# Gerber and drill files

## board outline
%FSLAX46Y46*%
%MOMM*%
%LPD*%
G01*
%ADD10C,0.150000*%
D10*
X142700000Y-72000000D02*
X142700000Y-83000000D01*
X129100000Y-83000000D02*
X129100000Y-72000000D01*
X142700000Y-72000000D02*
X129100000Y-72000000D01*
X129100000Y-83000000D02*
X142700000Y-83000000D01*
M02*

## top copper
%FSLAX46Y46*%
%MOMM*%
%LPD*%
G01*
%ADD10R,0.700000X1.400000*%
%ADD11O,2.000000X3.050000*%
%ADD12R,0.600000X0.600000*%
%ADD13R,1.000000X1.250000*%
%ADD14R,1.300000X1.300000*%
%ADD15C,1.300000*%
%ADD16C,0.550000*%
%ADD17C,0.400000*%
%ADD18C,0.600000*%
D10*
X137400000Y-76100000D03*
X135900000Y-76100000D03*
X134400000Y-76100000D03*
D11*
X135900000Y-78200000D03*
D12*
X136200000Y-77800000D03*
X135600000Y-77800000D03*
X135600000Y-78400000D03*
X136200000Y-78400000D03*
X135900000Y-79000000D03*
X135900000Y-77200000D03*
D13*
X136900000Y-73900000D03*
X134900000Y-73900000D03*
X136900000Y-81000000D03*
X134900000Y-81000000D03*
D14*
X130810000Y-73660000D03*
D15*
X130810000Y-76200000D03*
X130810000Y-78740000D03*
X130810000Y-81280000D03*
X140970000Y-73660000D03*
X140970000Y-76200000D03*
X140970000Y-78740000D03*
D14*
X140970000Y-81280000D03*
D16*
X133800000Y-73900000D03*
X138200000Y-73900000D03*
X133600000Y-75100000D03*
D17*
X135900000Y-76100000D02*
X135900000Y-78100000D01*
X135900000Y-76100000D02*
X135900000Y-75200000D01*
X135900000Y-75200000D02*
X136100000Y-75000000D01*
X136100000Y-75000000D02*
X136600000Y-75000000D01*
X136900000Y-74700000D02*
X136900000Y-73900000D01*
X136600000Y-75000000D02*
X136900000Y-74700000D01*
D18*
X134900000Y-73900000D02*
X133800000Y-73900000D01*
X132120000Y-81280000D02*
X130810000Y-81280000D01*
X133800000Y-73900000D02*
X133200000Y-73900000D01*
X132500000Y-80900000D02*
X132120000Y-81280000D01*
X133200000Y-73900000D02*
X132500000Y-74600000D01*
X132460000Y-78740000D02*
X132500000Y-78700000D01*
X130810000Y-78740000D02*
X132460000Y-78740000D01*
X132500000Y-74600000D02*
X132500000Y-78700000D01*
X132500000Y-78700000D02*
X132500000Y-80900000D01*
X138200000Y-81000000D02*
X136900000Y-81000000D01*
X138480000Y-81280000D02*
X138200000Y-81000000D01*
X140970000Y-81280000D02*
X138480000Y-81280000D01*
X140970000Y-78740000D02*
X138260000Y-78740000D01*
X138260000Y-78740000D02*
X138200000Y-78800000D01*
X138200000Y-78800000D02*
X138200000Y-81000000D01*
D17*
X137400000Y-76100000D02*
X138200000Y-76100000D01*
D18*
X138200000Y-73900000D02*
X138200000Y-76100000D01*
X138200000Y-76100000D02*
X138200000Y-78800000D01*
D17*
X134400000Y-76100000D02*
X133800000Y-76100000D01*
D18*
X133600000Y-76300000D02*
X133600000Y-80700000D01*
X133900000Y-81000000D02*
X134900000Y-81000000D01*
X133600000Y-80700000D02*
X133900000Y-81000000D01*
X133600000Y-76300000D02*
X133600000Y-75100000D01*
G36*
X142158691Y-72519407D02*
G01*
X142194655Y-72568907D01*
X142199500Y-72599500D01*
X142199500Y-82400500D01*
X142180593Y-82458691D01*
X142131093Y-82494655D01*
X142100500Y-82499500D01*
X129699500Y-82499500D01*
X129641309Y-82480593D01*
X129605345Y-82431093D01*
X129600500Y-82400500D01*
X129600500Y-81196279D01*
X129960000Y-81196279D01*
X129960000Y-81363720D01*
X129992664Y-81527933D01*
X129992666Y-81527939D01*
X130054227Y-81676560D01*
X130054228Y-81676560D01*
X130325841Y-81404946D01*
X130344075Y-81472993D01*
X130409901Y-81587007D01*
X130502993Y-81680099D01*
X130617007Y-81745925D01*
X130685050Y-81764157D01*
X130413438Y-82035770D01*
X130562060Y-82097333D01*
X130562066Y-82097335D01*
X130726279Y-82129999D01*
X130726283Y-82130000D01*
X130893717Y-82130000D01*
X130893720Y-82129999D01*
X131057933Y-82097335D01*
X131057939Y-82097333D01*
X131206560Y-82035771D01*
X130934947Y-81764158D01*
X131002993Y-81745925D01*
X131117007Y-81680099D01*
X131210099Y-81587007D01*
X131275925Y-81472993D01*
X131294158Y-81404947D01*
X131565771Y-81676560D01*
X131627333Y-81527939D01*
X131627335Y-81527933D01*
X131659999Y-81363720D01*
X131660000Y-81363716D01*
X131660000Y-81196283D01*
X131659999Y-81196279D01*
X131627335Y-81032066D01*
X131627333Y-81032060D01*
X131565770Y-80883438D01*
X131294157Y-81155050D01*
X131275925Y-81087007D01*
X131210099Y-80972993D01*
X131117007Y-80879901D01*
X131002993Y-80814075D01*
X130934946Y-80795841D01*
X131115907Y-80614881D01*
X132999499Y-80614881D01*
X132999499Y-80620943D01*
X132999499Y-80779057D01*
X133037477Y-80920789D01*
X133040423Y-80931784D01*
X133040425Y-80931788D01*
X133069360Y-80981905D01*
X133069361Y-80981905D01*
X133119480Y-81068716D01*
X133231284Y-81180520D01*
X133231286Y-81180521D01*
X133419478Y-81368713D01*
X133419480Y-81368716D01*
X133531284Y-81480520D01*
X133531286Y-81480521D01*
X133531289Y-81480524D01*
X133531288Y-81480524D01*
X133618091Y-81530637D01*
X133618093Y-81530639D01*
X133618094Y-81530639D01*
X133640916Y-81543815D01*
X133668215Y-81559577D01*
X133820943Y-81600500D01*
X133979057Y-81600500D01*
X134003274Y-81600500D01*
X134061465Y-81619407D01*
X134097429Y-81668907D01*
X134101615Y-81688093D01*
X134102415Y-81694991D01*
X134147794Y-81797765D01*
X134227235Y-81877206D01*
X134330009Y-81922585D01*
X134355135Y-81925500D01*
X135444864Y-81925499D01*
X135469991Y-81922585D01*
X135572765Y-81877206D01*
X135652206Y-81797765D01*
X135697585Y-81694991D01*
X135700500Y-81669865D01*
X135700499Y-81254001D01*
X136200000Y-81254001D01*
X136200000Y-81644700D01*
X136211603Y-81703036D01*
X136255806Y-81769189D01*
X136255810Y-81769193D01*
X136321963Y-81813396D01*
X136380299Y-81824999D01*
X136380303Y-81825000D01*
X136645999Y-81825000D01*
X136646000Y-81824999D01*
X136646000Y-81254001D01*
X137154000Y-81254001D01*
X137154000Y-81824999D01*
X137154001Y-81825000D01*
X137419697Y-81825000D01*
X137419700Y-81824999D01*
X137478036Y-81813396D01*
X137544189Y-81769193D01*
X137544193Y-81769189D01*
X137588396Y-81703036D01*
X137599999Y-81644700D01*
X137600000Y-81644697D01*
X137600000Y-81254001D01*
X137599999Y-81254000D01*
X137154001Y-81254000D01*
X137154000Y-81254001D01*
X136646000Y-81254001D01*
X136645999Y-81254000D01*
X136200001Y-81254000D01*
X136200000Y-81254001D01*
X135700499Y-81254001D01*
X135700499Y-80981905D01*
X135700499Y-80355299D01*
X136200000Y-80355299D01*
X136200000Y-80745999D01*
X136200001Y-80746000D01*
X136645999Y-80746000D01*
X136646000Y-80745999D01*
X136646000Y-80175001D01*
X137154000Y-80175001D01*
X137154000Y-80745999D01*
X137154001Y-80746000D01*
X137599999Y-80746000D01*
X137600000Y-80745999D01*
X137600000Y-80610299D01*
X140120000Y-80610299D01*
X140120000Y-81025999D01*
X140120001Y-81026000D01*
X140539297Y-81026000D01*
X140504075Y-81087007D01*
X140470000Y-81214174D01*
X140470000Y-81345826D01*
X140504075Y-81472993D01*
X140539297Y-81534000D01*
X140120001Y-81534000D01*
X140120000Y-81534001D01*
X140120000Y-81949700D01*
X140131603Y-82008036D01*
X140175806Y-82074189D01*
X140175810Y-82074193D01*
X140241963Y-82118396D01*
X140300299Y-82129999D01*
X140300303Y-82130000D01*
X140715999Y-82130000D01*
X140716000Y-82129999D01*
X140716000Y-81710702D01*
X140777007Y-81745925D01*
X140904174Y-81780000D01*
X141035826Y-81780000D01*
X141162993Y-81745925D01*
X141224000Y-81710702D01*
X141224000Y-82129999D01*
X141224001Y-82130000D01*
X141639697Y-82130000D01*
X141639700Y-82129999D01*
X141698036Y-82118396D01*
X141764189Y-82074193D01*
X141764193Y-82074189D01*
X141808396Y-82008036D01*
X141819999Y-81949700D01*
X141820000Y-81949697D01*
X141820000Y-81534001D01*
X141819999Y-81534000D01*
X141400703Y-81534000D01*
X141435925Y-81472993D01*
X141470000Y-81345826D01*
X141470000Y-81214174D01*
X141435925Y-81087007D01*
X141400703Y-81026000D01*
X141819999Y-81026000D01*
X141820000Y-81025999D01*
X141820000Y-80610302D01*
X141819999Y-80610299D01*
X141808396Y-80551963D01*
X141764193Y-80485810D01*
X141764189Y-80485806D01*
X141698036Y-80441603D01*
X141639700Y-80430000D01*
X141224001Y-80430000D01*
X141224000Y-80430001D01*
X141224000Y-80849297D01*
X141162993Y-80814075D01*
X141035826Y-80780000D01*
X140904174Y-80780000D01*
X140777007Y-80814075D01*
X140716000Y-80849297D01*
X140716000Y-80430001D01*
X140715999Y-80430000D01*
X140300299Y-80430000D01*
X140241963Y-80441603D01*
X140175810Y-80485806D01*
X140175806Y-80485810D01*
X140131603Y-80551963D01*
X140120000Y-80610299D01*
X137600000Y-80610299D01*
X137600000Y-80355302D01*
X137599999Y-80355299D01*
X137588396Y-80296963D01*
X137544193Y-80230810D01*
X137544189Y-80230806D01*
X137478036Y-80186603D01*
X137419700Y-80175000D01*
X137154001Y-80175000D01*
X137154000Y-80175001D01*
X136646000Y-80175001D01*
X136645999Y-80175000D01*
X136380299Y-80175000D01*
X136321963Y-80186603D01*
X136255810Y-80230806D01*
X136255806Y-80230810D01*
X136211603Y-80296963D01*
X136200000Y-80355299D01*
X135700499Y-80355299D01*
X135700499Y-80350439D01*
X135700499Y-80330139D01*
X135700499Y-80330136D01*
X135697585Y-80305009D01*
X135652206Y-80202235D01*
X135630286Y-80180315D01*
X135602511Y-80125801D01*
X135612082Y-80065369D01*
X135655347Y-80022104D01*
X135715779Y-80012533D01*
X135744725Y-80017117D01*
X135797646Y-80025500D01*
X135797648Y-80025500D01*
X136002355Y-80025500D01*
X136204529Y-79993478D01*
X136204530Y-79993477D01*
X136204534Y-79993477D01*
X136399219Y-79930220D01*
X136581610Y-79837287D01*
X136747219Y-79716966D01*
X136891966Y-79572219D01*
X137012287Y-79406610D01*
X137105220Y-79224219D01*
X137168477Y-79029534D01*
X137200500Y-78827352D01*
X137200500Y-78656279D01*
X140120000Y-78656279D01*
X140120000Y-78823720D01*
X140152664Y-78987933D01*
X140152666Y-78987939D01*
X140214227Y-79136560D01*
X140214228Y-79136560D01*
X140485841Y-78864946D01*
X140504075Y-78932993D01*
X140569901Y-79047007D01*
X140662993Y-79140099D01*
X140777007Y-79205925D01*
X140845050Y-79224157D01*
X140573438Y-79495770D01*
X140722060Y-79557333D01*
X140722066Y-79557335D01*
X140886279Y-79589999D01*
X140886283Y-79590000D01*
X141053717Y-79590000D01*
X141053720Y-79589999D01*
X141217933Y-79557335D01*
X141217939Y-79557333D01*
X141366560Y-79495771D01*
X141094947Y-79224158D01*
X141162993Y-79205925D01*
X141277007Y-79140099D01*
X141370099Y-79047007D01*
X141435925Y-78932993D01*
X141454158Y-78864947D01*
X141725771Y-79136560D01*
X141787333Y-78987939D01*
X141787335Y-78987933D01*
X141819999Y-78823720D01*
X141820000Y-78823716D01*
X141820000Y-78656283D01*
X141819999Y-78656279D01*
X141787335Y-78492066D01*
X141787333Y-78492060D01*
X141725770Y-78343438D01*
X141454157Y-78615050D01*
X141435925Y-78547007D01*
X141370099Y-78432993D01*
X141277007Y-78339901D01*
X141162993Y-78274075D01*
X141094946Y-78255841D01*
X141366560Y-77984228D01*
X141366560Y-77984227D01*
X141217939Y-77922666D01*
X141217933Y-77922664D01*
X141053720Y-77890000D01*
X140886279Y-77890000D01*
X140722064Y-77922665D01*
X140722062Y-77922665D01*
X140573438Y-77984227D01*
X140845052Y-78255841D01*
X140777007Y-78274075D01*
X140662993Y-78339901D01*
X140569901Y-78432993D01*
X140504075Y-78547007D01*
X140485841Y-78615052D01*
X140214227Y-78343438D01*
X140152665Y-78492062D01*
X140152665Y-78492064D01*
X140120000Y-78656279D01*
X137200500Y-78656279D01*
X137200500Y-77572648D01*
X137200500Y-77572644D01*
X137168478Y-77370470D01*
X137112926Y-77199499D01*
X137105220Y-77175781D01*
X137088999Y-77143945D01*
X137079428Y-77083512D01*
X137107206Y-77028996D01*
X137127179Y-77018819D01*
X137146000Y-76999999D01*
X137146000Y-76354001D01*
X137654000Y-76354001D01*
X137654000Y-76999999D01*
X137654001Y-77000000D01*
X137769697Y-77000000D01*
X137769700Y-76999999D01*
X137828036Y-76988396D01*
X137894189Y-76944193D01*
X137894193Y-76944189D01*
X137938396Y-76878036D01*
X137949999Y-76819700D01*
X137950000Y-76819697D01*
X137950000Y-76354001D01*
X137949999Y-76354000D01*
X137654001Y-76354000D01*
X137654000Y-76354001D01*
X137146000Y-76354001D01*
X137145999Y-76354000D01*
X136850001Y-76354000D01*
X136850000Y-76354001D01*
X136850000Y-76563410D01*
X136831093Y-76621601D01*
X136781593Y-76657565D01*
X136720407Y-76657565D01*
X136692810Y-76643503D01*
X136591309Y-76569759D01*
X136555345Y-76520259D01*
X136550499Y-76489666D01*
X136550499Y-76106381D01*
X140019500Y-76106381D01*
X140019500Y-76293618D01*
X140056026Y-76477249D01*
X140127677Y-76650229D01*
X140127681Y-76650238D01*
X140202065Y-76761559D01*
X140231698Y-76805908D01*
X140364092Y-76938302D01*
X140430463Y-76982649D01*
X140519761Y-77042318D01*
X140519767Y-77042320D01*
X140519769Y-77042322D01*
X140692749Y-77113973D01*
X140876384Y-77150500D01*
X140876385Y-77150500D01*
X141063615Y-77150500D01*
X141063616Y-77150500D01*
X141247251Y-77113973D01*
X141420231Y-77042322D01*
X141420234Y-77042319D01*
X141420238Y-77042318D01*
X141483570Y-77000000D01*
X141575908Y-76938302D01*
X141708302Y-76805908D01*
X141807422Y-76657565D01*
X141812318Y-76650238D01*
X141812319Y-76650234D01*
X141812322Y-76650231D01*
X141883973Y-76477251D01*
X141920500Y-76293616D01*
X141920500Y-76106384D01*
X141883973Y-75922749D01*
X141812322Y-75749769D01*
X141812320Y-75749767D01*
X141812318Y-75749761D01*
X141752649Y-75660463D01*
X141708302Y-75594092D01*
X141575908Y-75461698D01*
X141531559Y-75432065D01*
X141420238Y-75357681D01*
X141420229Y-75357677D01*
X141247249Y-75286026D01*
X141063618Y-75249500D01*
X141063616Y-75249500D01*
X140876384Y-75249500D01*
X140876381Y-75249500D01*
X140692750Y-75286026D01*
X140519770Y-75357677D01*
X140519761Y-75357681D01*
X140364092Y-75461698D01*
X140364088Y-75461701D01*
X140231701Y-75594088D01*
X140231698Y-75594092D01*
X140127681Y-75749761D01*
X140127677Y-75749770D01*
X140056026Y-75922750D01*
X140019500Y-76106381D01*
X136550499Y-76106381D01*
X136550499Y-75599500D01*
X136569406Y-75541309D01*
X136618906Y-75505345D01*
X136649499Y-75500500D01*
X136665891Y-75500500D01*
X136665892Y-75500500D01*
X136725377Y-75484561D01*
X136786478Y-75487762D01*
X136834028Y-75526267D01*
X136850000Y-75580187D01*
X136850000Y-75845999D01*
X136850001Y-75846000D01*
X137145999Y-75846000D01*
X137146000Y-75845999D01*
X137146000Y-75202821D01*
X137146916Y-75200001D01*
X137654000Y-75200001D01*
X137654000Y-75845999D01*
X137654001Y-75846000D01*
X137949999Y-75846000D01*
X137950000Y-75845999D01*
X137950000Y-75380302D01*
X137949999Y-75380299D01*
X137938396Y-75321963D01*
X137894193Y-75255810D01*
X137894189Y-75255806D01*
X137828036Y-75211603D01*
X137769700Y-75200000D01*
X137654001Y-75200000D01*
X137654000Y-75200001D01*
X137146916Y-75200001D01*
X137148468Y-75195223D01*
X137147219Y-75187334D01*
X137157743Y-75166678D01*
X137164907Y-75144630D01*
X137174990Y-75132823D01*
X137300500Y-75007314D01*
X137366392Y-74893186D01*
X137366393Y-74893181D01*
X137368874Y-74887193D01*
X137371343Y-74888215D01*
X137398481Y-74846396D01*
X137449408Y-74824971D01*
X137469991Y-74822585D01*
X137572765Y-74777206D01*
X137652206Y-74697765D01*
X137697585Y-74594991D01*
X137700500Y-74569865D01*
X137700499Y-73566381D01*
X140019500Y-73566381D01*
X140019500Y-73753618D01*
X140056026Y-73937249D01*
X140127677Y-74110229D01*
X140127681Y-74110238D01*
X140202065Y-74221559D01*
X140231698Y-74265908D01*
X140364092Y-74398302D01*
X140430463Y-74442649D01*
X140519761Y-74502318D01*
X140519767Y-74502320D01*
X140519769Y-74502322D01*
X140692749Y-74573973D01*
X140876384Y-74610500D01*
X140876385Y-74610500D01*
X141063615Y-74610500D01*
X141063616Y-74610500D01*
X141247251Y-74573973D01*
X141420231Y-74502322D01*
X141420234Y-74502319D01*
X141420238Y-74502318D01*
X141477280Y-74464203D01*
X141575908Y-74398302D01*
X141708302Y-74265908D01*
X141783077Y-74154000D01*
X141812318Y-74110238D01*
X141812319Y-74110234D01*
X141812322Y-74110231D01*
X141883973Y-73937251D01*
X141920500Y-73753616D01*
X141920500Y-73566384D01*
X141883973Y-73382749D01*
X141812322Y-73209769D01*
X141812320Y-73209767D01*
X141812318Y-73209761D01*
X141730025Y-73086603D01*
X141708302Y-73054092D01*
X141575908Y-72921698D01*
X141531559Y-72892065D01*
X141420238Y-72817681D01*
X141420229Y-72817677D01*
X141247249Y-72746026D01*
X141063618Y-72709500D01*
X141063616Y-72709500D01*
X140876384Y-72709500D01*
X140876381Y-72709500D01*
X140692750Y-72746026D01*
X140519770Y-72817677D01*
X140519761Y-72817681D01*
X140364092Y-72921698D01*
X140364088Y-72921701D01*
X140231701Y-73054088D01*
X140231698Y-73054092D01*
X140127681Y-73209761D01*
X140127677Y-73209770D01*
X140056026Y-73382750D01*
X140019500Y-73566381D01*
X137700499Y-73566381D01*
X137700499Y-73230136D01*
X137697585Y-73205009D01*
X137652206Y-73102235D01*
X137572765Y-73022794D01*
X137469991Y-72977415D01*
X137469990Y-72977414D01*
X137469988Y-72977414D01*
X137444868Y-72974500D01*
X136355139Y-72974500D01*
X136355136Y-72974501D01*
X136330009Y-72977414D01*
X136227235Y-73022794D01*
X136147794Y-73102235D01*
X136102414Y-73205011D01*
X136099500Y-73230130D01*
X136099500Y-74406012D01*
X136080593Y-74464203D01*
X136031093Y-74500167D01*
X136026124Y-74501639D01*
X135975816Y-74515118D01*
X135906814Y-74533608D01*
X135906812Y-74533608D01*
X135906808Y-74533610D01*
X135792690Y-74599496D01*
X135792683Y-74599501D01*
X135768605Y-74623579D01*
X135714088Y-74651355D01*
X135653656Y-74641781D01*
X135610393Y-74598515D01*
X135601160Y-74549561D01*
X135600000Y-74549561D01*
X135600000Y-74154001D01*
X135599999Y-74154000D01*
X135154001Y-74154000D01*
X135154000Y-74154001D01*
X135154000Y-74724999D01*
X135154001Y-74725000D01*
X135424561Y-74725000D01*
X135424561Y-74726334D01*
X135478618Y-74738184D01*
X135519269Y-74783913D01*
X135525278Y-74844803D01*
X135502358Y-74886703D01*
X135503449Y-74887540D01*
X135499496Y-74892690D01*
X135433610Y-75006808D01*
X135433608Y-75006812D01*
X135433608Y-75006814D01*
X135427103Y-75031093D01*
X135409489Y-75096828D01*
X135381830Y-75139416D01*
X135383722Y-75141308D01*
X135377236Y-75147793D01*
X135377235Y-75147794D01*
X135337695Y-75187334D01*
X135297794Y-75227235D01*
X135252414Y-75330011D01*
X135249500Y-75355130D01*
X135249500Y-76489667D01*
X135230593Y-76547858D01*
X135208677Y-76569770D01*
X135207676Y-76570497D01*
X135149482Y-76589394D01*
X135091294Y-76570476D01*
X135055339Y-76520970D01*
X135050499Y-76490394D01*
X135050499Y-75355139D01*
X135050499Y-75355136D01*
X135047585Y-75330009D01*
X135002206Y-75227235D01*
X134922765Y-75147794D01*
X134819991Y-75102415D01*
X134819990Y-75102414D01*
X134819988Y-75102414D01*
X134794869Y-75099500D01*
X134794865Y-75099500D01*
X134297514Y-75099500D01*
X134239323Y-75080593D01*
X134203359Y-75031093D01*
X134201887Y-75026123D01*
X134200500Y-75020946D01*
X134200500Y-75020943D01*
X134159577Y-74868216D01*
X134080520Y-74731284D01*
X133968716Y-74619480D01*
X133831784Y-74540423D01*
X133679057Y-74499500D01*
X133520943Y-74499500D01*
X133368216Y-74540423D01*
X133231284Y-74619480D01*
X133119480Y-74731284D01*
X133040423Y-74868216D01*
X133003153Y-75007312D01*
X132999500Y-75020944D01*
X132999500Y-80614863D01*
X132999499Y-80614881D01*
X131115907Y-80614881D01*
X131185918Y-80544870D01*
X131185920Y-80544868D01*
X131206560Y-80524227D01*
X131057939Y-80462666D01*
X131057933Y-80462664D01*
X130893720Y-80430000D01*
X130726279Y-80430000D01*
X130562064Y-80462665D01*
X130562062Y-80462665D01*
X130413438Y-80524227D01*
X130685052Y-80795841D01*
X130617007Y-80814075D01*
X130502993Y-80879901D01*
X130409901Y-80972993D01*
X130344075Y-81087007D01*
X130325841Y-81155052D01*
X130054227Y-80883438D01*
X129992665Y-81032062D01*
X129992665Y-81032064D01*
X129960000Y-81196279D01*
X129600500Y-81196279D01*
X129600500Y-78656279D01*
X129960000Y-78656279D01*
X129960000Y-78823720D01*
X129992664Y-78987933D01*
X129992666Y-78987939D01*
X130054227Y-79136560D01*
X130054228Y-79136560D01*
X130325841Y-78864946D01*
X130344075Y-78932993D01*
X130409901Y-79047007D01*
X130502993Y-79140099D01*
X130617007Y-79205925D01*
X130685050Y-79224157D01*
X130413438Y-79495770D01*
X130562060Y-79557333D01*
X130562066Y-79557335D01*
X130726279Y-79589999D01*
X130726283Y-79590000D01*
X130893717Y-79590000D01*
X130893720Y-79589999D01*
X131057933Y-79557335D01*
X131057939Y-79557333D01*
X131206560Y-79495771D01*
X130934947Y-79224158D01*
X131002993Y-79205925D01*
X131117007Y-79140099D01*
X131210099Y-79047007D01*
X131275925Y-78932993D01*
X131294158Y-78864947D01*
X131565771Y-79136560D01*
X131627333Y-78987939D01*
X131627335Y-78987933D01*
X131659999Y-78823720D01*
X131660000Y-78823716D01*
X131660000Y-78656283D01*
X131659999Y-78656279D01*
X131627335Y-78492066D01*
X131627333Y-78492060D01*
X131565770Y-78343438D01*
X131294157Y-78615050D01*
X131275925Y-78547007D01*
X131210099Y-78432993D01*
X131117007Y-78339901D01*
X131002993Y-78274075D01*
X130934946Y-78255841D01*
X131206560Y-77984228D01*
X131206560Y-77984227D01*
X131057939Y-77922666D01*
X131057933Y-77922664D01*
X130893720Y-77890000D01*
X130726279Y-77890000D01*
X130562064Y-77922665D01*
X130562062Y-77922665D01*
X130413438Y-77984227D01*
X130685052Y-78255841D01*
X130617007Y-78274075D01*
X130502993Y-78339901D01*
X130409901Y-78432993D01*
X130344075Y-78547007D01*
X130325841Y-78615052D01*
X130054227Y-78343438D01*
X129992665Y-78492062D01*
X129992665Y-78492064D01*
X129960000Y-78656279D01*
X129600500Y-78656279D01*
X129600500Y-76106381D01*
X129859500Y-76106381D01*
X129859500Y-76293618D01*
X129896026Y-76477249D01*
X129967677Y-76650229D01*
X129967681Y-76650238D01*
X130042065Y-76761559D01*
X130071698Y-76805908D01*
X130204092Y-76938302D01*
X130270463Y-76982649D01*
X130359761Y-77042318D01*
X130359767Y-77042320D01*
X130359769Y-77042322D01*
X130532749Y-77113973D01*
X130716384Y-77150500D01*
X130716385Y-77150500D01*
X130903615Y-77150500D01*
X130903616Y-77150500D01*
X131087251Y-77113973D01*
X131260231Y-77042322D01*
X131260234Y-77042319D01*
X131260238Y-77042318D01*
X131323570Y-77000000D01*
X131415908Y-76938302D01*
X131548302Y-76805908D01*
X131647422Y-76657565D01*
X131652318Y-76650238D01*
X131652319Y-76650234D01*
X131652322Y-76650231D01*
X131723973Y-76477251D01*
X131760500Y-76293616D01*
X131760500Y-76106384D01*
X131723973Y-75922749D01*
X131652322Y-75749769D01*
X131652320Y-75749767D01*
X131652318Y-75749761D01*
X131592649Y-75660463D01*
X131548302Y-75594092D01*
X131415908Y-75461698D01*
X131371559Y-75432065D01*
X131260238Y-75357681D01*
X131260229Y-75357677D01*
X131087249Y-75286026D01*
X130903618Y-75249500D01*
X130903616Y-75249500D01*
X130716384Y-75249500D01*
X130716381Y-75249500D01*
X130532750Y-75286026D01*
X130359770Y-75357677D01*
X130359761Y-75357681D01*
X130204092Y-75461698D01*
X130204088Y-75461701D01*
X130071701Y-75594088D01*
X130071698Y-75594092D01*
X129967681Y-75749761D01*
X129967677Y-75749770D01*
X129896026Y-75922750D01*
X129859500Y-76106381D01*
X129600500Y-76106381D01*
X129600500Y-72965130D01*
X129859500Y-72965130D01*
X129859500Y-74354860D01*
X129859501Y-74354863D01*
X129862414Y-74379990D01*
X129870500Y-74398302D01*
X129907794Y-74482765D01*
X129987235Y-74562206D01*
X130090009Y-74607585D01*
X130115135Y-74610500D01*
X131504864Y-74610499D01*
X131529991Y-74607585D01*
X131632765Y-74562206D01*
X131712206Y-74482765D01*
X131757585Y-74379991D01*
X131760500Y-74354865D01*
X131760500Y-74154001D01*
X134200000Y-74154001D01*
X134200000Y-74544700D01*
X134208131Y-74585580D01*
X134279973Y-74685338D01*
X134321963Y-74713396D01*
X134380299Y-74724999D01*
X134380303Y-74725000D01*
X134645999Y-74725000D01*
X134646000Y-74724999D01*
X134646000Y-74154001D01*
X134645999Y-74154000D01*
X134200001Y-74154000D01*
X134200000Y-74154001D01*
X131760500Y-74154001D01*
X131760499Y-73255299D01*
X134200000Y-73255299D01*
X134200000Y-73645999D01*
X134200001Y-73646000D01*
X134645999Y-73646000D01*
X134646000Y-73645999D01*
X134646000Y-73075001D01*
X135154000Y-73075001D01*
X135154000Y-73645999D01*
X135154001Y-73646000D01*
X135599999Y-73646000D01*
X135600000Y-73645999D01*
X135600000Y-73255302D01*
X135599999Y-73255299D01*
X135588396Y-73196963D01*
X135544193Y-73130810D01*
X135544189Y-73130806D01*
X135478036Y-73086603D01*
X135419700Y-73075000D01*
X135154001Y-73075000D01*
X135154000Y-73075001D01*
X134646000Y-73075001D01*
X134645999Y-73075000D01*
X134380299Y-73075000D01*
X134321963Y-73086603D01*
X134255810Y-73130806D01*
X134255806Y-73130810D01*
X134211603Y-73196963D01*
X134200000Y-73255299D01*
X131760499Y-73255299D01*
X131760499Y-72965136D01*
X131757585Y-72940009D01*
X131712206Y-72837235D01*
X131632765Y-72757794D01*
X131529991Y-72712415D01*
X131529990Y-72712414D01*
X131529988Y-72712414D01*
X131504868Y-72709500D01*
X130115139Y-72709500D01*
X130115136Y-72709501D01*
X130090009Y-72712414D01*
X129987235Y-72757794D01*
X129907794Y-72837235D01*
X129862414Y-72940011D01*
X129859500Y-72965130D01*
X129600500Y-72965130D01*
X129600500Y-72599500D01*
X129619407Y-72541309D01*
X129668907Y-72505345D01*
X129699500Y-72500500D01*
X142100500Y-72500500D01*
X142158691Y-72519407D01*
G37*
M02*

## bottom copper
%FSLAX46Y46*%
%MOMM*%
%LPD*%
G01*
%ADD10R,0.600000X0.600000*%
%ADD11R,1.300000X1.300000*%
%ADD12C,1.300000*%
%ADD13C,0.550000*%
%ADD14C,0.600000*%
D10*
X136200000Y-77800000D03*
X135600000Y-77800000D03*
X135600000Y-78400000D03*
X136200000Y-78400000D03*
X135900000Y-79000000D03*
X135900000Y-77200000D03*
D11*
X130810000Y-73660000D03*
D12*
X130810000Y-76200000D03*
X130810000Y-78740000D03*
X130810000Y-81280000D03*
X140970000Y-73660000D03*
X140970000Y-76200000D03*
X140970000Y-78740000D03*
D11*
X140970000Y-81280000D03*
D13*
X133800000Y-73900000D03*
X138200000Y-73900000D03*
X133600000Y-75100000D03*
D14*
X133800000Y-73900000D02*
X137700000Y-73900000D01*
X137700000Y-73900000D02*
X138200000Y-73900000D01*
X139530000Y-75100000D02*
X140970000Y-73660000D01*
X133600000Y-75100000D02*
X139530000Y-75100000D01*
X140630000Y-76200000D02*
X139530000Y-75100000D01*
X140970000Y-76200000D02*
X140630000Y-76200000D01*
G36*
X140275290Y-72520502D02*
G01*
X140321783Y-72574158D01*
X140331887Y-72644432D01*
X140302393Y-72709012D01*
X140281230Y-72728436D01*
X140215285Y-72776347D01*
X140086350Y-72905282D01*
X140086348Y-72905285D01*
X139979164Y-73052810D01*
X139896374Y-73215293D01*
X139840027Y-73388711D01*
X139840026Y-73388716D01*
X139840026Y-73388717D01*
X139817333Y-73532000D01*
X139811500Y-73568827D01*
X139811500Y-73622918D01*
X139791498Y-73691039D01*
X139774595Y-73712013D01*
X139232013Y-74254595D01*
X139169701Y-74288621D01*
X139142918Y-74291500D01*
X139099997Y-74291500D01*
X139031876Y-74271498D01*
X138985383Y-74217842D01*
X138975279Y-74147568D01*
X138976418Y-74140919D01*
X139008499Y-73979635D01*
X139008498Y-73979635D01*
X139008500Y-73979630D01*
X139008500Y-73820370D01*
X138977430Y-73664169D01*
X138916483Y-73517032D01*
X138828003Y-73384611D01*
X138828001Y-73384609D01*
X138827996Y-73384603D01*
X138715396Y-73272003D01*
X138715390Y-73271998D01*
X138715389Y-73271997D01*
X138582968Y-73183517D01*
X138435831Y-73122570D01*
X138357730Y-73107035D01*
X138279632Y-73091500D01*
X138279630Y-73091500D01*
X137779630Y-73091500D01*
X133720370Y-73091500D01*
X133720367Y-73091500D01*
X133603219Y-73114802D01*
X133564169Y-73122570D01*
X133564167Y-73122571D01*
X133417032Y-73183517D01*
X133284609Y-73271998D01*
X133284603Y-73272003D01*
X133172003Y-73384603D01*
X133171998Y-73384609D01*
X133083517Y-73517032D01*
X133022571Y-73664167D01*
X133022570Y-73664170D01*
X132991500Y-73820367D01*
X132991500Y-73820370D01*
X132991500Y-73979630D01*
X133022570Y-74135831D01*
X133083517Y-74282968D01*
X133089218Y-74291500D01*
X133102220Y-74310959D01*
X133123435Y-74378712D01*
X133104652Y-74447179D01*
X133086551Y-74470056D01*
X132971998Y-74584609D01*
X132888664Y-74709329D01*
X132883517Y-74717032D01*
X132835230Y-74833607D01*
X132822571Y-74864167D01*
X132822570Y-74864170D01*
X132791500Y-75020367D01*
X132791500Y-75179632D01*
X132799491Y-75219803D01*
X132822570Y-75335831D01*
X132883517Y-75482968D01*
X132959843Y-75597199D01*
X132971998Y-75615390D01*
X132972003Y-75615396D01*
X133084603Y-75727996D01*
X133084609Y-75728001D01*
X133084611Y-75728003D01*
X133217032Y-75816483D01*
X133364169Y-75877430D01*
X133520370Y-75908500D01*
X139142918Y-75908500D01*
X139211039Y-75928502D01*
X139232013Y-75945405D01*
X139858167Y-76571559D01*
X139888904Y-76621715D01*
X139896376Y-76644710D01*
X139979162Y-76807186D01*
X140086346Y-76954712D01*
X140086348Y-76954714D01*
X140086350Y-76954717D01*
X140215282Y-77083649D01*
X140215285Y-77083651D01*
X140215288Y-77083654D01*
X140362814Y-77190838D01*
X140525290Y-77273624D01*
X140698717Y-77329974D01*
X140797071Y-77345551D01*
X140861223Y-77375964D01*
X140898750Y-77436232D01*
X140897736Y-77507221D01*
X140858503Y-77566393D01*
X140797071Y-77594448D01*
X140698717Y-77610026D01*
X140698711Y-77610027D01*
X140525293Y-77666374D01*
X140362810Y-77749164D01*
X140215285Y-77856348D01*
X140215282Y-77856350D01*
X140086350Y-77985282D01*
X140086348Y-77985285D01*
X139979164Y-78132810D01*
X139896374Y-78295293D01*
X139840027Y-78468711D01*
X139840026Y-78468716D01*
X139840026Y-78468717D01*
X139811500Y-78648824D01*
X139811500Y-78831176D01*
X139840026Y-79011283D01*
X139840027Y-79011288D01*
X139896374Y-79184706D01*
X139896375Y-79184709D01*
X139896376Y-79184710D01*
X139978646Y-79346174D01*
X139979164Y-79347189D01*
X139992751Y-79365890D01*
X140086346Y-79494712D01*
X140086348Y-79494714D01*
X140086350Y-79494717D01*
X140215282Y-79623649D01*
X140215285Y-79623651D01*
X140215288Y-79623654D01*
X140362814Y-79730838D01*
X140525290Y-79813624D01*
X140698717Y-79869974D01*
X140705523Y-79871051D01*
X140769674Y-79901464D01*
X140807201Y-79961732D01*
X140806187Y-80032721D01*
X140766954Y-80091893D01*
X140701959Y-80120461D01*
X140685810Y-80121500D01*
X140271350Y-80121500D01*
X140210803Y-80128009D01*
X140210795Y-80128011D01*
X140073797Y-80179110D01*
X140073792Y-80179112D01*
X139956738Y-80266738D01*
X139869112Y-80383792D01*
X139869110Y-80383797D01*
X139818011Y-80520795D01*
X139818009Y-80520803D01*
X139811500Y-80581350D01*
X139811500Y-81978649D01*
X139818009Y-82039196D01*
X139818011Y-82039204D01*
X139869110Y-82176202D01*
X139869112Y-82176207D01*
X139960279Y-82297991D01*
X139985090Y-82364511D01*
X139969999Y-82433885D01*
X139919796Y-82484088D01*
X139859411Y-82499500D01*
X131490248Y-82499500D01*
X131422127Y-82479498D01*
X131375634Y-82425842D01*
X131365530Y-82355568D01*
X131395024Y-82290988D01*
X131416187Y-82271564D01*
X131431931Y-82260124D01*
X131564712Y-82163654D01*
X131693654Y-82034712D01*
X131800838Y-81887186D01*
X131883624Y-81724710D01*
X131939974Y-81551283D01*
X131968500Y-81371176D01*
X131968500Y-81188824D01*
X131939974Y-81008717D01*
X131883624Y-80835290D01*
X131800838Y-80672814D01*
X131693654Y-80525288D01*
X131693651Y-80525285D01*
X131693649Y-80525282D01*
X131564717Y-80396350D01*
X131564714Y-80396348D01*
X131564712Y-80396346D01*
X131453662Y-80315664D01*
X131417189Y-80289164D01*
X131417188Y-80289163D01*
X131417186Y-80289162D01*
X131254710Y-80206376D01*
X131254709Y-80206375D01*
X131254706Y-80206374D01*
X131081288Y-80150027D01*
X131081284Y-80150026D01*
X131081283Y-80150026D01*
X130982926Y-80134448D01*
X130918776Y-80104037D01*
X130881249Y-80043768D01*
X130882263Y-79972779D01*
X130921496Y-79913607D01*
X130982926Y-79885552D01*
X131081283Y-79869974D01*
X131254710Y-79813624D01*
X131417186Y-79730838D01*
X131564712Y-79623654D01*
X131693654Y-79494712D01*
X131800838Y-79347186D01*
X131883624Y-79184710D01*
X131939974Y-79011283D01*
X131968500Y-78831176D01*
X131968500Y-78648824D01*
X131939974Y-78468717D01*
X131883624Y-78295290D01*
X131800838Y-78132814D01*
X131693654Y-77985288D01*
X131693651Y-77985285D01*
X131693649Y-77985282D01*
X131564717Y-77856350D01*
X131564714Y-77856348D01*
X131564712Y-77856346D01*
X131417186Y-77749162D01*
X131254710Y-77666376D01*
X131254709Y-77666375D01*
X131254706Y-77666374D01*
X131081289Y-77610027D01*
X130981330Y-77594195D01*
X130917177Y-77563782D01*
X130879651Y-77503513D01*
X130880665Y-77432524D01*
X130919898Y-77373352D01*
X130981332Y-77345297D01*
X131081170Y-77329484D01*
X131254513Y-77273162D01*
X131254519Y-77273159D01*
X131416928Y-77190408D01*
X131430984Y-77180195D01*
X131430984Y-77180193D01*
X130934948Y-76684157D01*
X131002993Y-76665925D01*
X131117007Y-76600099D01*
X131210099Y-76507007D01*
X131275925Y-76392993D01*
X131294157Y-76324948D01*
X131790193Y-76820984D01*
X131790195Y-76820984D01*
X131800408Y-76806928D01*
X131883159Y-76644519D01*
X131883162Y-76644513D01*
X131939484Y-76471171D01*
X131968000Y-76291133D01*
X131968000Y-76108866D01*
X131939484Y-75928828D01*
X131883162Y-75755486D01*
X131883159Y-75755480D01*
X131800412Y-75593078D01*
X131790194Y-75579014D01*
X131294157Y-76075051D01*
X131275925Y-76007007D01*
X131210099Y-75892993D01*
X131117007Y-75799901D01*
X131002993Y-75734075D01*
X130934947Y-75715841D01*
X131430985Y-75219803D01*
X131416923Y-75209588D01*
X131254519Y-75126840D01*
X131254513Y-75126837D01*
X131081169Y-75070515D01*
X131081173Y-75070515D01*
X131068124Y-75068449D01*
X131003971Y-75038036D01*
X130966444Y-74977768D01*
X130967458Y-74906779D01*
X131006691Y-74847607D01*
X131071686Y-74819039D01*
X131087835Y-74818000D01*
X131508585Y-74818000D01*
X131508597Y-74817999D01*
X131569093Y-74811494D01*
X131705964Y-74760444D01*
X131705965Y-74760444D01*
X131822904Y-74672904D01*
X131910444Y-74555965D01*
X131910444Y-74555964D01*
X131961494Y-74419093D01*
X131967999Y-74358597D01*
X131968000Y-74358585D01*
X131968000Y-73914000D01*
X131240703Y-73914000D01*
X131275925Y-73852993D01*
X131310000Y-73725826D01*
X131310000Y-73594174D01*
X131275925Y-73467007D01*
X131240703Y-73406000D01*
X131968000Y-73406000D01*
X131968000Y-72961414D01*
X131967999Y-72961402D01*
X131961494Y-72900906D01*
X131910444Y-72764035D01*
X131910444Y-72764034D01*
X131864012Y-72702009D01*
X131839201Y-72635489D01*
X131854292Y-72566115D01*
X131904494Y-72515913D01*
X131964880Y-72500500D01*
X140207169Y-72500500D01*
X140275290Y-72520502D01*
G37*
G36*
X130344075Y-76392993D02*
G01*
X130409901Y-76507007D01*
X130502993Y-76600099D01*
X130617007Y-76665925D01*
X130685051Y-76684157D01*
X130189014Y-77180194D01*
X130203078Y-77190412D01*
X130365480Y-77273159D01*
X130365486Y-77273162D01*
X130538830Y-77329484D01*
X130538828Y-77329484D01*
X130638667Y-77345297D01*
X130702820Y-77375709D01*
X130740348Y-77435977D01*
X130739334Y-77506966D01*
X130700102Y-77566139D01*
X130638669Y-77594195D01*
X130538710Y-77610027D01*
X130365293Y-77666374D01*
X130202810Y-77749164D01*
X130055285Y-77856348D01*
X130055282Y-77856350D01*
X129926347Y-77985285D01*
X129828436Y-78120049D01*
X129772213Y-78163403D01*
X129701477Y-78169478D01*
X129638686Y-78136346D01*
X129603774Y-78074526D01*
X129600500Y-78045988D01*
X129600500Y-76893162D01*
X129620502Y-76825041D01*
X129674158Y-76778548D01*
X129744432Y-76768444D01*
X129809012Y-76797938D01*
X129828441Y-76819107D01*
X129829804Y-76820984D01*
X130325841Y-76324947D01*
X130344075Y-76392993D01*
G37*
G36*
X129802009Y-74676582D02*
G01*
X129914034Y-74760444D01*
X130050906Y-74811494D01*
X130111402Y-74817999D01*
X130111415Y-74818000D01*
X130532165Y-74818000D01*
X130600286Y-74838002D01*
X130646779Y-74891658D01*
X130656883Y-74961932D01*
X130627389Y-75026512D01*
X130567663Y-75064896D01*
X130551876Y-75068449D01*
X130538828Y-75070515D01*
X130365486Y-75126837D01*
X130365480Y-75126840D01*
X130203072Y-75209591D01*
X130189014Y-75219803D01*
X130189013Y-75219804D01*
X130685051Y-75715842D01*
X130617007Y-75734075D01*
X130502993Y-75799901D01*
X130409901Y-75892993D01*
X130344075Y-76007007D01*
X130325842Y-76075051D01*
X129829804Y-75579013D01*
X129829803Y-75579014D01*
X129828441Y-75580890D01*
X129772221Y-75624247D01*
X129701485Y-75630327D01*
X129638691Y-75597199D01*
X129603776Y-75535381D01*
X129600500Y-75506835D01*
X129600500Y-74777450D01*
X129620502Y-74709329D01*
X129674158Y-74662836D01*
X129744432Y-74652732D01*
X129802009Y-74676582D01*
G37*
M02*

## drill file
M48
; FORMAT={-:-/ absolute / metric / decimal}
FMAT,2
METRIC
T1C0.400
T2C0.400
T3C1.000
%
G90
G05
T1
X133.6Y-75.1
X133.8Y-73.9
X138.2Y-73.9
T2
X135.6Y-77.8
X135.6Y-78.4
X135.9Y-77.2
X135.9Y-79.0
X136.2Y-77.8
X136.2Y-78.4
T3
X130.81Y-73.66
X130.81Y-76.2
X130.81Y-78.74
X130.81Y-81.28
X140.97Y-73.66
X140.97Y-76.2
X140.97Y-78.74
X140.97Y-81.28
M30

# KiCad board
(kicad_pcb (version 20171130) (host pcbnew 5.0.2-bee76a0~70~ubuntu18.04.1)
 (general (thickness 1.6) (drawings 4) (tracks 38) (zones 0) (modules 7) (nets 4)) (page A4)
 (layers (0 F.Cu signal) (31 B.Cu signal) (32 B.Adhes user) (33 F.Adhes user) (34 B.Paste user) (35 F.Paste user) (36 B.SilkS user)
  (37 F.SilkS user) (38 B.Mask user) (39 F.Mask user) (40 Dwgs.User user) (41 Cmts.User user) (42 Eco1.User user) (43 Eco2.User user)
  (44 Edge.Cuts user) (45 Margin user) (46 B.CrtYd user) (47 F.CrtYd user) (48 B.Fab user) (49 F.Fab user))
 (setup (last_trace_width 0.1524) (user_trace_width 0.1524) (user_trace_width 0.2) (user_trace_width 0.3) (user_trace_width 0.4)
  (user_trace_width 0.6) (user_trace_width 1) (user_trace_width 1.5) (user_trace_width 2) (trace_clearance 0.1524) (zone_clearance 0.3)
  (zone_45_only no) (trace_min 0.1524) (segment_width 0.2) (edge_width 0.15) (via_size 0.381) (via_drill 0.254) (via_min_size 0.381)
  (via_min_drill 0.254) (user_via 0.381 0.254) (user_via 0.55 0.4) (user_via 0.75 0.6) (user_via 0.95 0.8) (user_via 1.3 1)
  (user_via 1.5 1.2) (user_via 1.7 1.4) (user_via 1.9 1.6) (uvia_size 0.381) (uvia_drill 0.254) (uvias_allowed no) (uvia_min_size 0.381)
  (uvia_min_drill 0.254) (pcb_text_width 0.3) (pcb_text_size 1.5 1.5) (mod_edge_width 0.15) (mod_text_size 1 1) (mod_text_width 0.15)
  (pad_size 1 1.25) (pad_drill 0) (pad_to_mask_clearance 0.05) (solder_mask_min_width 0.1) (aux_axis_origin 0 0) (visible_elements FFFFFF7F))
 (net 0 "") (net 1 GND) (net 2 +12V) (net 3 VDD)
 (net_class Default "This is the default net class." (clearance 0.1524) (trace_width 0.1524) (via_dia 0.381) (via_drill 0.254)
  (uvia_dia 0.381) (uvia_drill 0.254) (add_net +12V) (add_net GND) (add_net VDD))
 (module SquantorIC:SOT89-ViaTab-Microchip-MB (layer F.Cu) (at 135.9 76.1 180)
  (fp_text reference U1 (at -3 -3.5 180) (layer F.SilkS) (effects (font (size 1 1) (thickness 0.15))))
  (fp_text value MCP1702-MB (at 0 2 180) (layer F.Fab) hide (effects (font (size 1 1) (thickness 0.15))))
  (pad 1 smd rect (at -1.5 0 180) (size 0.7 1.4) (layers F.Cu F.Paste F.Mask) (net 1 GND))
  (pad 2 smd rect (at 0 0 180) (size 0.7 1.4) (layers F.Cu F.Paste F.Mask) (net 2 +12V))
  (pad 3 smd rect (at 1.5 0 180) (size 0.7 1.4) (layers F.Cu F.Paste F.Mask) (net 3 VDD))
  (pad TAB smd oval (at 0 -2.1 180) (size 2 3.05) (layers F.Cu F.Paste F.Mask) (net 2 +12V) (zone_connect 2))
  (pad TAB thru_hole rect (at -0.3 -1.7 180) (size 0.6 0.6) (drill 0.4) (layers *.Cu *.Mask) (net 2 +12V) (zone_connect 2))
  (pad TAB thru_hole rect (at 0.3 -1.7 180) (size 0.6 0.6) (drill 0.4) (layers *.Cu *.Mask) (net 2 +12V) (zone_connect 2))
  (pad TAB thru_hole rect (at 0.3 -2.3 180) (size 0.6 0.6) (drill 0.4) (layers *.Cu *.Mask) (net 2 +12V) (zone_connect 2))
  (pad TAB thru_hole rect (at -0.3 -2.3 180) (size 0.6 0.6) (drill 0.4) (layers *.Cu *.Mask) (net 2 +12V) (zone_connect 2))
  (pad TAB thru_hole rect (at 0 -2.9 180) (size 0.6 0.6) (drill 0.4) (layers *.Cu *.Mask) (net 2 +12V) (zone_connect 2))
  (pad TAB thru_hole rect (at 0 -1.1 180) (size 0.6 0.6) (drill 0.4) (layers *.Cu *.Mask) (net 2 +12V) (zone_connect 2)))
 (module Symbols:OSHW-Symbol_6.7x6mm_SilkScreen (layer B.Cu) (at 135.9 75.3 180)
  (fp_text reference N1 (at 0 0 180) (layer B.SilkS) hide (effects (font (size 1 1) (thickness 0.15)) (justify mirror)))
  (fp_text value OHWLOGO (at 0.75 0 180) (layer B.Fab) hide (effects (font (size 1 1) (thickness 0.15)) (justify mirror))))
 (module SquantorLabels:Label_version (layer B.Cu) (at 135.3 80.01 90)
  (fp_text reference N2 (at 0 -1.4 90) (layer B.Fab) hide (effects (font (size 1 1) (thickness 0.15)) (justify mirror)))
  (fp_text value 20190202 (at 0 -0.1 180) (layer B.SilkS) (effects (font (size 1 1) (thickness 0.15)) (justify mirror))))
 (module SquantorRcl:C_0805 (layer F.Cu) (at 135.9 73.9 180)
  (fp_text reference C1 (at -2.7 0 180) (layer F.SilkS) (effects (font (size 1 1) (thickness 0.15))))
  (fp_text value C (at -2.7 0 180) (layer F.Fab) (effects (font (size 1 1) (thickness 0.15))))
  (pad 1 smd rect (at -1 0 180) (size 1 1.25) (layers F.Cu F.Paste F.Mask) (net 2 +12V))
  (pad 2 smd rect (at 1 0 180) (size 1 1.25) (layers F.Cu F.Paste F.Mask) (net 1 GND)))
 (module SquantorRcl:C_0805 (layer F.Cu) (at 135.9 81)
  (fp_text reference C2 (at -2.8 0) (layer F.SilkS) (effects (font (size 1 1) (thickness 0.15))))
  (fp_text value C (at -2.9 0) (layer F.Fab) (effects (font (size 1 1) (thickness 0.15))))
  (pad 2 smd rect (at 1 0) (size 1 1.25) (layers F.Cu F.Paste F.Mask) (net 1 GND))
  (pad 1 smd rect (at -1 0) (size 1 1.25) (layers F.Cu F.Paste F.Mask) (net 3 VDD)))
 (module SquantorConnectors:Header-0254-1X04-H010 (layer F.Cu) (at 130.81 77.47 270)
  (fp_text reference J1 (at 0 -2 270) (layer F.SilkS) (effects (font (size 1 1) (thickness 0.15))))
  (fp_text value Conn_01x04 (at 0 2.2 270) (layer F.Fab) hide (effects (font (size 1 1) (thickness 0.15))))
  (pad 1 thru_hole rect (at -3.81 0 90) (size 1.3 1.3) (drill 1) (layers *.Cu *.Mask) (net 2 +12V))
  (pad 2 thru_hole circle (at -1.27 0 90) (size 1.3 1.3) (drill 1) (layers *.Cu *.Mask) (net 2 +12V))
  (pad 3 thru_hole circle (at 1.27 0 90) (size 1.3 1.3) (drill 1) (layers *.Cu *.Mask) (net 1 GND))
  (pad 4 thru_hole circle (at 3.81 0 90) (size 1.3 1.3) (drill 1) (layers *.Cu *.Mask) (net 1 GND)))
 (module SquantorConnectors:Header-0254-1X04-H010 (layer F.Cu) (at 140.97 77.47 90)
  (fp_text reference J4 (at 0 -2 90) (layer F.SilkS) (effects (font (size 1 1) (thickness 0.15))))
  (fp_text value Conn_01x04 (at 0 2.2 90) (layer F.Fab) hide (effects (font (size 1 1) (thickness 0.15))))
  (pad 4 thru_hole circle (at 3.81 0 270) (size 1.3 1.3) (drill 1) (layers *.Cu *.Mask) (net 3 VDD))
  (pad 3 thru_hole circle (at 1.27 0 270) (size 1.3 1.3) (drill 1) (layers *.Cu *.Mask) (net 3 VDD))
  (pad 2 thru_hole circle (at -1.27 0 270) (size 1.3 1.3) (drill 1) (layers *.Cu *.Mask) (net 1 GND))
  (pad 1 thru_hole rect (at -3.81 0 270) (size 1.3 1.3) (drill 1) (layers *.Cu *.Mask) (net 1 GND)))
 (gr_line (start 142.7 72) (end 142.7 83) (layer Edge.Cuts) (width 0.15))
 (gr_line (start 129.1 83) (end 129.1 72) (layer Edge.Cuts) (width 0.15))
 (gr_line (start 142.7 72) (end 129.1 72) (layer Edge.Cuts) (width 0.15))
 (gr_line (start 129.1 83) (end 142.7 83) (layer Edge.Cuts) (width 0.15))
 (segment (start 135.9 76.1) (end 135.9 78.1) (width 0.4) (layer F.Cu) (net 2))
 (segment (start 135.9 76.1) (end 135.9 75.2) (width 0.4) (layer F.Cu) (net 2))
 (segment (start 135.9 75.2) (end 136.1 75) (width 0.4) (layer F.Cu) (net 2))
 (segment (start 136.1 75) (end 136.6 75) (width 0.4) (layer F.Cu) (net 2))
 (segment (start 136.9 74.7) (end 136.9 73.9) (width 0.4) (layer F.Cu) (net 2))
 (segment (start 136.6 75) (end 136.9 74.7) (width 0.4) (layer F.Cu) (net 2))
 (segment (start 134.9 73.9) (end 133.8 73.9) (width 0.6) (layer F.Cu) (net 1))
 (via (at 133.8 73.9) (size 0.55) (drill 0.4) (layers F.Cu B.Cu) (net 1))
 (segment (start 133.8 73.9) (end 137.7 73.9) (width 0.6) (layer B.Cu) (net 1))
 (segment (start 132.12 81.28) (end 130.81 81.28) (width 0.6) (layer F.Cu) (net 1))
 (segment (start 133.8 73.9) (end 133.2 73.9) (width 0.6) (layer F.Cu) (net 1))
 (segment (start 132.5 80.9) (end 132.12 81.28) (width 0.6) (layer F.Cu) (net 1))
 (segment (start 133.2 73.9) (end 132.5 74.6) (width 0.6) (layer F.Cu) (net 1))
 (segment (start 132.46 78.74) (end 132.5 78.7) (width 0.6) (layer F.Cu) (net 1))
 (segment (start 130.81 78.74) (end 132.46 78.74) (width 0.6) (layer F.Cu) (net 1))
 (segment (start 132.5 74.6) (end 132.5 78.7) (width 0.6) (layer F.Cu) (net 1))
 (segment (start 132.5 78.7) (end 132.5 80.9) (width 0.6) (layer F.Cu) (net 1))
 (segment (start 137.7 73.9) (end 138.2 73.9) (width 0.6) (layer B.Cu) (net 1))
 (via (at 138.2 73.9) (size 0.55) (drill 0.4) (layers F.Cu B.Cu) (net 1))
 (segment (start 138.2 81) (end 136.9 81) (width 0.6) (layer F.Cu) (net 1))
 (segment (start 138.48 81.28) (end 138.2 81) (width 0.6) (layer F.Cu) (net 1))
 (segment (start 140.97 81.28) (end 138.48 81.28) (width 0.6) (layer F.Cu) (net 1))
 (segment (start 140.97 78.74) (end 138.26 78.74) (width 0.6) (layer F.Cu) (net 1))
 (segment (start 138.26 78.74) (end 138.2 78.8) (width 0.6) (layer F.Cu) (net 1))
 (segment (start 138.2 78.8) (end 138.2 81) (width 0.6) (layer F.Cu) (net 1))
 (segment (start 137.4 76.1) (end 138.2 76.1) (width 0.4) (layer F.Cu) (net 1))
 (segment (start 138.2 73.9) (end 138.2 76.1) (width 0.6) (layer F.Cu) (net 1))
 (segment (start 138.2 76.1) (end 138.2 78.8) (width 0.6) (layer F.Cu) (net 1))
 (segment (start 134.4 76.1) (end 133.8 76.1) (width 0.4) (layer F.Cu) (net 3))
 (segment (start 133.6 76.3) (end 133.6 80.7) (width 0.6) (layer F.Cu) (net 3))
 (segment (start 133.9 81) (end 134.9 81) (width 0.6) (layer F.Cu) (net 3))
 (segment (start 133.6 80.7) (end 133.9 81) (width 0.6) (layer F.Cu) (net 3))
 (segment (start 133.6 76.3) (end 133.6 75.1) (width 0.6) (layer F.Cu) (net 3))
 (via (at 133.6 75.1) (size 0.55) (drill 0.4) (layers F.Cu B.Cu) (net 3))
 (segment (start 139.53 75.1) (end 140.97 73.66) (width 0.6) (layer B.Cu) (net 3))
 (segment (start 133.6 75.1) (end 139.53 75.1) (width 0.6) (layer B.Cu) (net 3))
 (segment (start 140.63 76.2) (end 139.53 75.1) (width 0.6) (layer B.Cu) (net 3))
 (segment (start 140.97 76.2) (end 140.63 76.2) (width 0.6) (layer B.Cu) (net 3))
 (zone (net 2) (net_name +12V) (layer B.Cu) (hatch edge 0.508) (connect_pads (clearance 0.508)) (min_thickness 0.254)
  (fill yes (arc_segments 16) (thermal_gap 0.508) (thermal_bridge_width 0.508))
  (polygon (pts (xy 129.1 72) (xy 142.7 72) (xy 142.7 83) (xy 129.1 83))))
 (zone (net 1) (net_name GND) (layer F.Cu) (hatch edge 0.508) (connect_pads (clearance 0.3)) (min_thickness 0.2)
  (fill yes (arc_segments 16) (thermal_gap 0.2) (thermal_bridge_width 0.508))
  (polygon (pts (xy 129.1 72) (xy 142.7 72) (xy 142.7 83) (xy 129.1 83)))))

